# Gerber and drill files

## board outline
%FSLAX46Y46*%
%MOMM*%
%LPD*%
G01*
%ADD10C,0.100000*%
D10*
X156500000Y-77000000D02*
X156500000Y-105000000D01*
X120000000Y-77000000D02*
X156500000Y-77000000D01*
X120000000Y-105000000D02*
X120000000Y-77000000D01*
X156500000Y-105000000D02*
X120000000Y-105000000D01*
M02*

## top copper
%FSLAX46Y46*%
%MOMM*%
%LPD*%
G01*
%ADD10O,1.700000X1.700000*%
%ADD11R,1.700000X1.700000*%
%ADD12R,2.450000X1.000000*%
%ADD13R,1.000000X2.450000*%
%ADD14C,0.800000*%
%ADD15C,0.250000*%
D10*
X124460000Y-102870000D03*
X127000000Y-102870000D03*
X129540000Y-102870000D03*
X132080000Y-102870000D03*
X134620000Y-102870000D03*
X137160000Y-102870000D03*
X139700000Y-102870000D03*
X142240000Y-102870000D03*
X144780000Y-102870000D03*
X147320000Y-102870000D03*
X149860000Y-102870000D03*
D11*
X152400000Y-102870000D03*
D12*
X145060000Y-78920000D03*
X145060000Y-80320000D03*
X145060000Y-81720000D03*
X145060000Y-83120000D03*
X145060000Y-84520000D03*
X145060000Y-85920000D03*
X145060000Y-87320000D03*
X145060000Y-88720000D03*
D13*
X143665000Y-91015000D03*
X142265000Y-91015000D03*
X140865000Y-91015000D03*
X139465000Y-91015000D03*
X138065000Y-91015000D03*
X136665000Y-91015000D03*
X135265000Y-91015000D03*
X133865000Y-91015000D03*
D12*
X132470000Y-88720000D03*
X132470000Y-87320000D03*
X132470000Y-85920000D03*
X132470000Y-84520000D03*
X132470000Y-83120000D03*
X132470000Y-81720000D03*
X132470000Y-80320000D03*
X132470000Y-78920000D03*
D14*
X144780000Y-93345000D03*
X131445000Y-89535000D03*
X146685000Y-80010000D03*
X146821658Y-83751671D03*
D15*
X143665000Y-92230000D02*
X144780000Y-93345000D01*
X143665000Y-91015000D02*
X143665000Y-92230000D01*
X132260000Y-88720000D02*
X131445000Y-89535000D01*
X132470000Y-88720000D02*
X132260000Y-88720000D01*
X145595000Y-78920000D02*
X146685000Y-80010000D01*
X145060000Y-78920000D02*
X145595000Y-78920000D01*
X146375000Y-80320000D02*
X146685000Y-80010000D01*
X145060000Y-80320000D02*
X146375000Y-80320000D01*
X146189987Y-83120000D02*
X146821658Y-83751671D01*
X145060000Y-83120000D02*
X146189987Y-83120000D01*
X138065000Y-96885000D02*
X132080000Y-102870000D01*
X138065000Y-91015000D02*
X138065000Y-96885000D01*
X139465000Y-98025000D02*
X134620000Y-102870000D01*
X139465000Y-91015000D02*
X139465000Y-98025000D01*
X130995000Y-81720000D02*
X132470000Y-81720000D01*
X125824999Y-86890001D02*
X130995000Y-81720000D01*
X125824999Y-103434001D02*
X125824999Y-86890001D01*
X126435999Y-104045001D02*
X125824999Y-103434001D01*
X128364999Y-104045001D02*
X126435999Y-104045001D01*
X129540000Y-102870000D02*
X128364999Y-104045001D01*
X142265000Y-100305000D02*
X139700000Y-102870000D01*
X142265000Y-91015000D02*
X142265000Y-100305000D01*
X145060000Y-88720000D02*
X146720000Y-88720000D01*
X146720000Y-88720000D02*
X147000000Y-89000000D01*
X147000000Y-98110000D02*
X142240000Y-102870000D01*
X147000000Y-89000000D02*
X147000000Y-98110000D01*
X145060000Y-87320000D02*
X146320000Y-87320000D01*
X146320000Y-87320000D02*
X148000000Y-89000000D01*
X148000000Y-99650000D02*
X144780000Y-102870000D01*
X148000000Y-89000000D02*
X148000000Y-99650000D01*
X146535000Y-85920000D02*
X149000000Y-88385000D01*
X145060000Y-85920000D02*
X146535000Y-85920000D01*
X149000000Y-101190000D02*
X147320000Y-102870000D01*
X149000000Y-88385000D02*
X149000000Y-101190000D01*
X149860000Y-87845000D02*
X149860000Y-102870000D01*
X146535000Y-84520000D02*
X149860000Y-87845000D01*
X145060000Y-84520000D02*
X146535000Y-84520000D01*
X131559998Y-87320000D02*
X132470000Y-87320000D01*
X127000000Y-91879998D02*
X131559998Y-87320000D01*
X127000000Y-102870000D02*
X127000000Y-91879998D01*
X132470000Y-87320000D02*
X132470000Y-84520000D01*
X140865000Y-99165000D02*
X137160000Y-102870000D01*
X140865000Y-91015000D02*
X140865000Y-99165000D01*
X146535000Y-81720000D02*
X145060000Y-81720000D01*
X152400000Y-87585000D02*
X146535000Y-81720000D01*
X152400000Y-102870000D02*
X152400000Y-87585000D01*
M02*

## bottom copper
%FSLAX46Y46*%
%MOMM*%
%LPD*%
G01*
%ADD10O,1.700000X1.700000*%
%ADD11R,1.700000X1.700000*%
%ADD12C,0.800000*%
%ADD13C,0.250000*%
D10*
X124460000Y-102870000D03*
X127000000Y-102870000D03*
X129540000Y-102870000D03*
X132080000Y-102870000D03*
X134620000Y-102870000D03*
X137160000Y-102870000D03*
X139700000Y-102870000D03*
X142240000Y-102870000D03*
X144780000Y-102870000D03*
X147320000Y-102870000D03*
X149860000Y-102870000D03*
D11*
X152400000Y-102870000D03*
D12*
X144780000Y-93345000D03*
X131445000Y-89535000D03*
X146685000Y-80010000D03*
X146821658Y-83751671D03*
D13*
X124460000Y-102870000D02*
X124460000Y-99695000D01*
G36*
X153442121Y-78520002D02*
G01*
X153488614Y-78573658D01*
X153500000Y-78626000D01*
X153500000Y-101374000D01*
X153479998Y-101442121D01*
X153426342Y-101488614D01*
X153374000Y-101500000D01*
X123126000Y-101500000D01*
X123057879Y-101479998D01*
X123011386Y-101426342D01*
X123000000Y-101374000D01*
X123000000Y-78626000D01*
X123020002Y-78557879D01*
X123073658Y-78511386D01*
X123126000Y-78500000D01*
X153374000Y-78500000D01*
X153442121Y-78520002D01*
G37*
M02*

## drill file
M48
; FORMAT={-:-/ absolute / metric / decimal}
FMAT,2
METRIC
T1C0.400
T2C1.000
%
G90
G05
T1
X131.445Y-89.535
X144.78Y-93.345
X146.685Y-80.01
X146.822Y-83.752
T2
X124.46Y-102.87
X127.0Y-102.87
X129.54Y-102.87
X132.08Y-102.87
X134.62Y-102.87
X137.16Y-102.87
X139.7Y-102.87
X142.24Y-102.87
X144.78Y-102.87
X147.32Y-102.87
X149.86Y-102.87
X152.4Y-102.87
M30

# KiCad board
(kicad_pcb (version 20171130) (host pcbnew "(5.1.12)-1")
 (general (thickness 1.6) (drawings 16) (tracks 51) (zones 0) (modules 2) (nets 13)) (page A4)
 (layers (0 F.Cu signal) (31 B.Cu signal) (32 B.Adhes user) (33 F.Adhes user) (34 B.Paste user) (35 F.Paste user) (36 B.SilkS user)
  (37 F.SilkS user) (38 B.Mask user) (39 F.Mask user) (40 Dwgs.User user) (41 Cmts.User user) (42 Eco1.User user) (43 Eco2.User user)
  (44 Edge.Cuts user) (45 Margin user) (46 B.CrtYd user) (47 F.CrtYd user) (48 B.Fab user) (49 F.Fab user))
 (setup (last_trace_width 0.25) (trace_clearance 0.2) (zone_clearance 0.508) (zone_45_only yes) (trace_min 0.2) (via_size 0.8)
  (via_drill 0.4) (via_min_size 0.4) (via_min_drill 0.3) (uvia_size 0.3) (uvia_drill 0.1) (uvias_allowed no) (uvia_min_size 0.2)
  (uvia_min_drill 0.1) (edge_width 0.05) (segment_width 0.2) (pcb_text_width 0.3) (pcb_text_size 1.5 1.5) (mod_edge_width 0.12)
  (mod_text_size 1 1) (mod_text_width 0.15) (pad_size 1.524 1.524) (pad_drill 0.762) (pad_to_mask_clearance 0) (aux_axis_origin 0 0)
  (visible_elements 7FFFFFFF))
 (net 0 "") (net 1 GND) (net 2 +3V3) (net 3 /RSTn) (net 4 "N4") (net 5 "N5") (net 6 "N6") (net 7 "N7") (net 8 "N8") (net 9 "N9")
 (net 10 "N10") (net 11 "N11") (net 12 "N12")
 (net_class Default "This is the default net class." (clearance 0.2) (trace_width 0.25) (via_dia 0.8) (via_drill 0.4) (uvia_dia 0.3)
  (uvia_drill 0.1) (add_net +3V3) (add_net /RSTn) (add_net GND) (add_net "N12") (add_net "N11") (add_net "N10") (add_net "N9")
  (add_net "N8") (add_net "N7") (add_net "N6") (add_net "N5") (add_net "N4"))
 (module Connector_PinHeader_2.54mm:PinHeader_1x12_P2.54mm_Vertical (layer F.Cu) (at 152.4 102.87 270)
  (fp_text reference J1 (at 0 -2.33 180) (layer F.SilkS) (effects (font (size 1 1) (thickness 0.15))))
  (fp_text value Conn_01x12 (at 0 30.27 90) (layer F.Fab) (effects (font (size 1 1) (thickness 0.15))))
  (pad 12 thru_hole oval (at 0 27.94 270) (size 1.7 1.7) (drill 1) (layers *.Cu *.Mask) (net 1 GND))
  (pad 11 thru_hole oval (at 0 25.4 270) (size 1.7 1.7) (drill 1) (layers *.Cu *.Mask) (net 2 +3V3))
  (pad 10 thru_hole oval (at 0 22.86 270) (size 1.7 1.7) (drill 1) (layers *.Cu *.Mask) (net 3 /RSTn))
  (pad 9 thru_hole oval (at 0 20.32 270) (size 1.7 1.7) (drill 1) (layers *.Cu *.Mask) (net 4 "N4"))
  (pad 8 thru_hole oval (at 0 17.78 270) (size 1.7 1.7) (drill 1) (layers *.Cu *.Mask) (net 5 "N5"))
  (pad 7 thru_hole oval (at 0 15.24 270) (size 1.7 1.7) (drill 1) (layers *.Cu *.Mask) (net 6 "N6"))
  (pad 6 thru_hole oval (at 0 12.7 270) (size 1.7 1.7) (drill 1) (layers *.Cu *.Mask) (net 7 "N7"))
  (pad 5 thru_hole oval (at 0 10.16 270) (size 1.7 1.7) (drill 1) (layers *.Cu *.Mask) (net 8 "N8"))
  (pad 4 thru_hole oval (at 0 7.62 270) (size 1.7 1.7) (drill 1) (layers *.Cu *.Mask) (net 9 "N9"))
  (pad 3 thru_hole oval (at 0 5.08 270) (size 1.7 1.7) (drill 1) (layers *.Cu *.Mask) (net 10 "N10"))
  (pad 2 thru_hole oval (at 0 2.54 270) (size 1.7 1.7) (drill 1) (layers *.Cu *.Mask) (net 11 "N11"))
  (pad 1 thru_hole rect (at 0 0 270) (size 1.7 1.7) (drill 1) (layers *.Cu *.Mask) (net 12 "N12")))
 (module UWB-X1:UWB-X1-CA (layer F.Cu) (at 138.765 83.82)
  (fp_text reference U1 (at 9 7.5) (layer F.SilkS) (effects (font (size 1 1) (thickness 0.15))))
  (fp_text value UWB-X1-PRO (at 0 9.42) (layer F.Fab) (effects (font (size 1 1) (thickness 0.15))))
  (pad 24 smd rect (at 6.295 -4.9 90) (size 1 2.45) (layers F.Cu F.Paste F.Mask) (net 1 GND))
  (pad 23 smd rect (at 6.295 -3.5 90) (size 1 2.45) (layers F.Cu F.Paste F.Mask) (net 1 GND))
  (pad 22 smd rect (at 6.295 -2.1 90) (size 1 2.45) (layers F.Cu F.Paste F.Mask) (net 12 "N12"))
  (pad 21 smd rect (at 6.295 -0.7 90) (size 1 2.45) (layers F.Cu F.Paste F.Mask) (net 1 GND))
  (pad 20 smd rect (at 6.295 0.7 90) (size 1 2.45) (layers F.Cu F.Paste F.Mask) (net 11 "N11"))
  (pad 19 smd rect (at 6.295 2.1 90) (size 1 2.45) (layers F.Cu F.Paste F.Mask) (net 10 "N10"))
  (pad 18 smd rect (at 6.295 3.5 90) (size 1 2.45) (layers F.Cu F.Paste F.Mask) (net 9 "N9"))
  (pad 17 smd rect (at 6.295 4.9 90) (size 1 2.45) (layers F.Cu F.Paste F.Mask) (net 8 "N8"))
  (pad 16 smd rect (at 4.9 7.195) (size 1 2.45) (layers F.Cu F.Paste F.Mask) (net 1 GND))
  (pad 15 smd rect (at 3.5 7.195) (size 1 2.45) (layers F.Cu F.Paste F.Mask) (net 7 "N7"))
  (pad 14 smd rect (at 2.1 7.195) (size 1 2.45) (layers F.Cu F.Paste F.Mask) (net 6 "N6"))
  (pad 13 smd rect (at 0.7 7.195) (size 1 2.45) (layers F.Cu F.Paste F.Mask) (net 5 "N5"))
  (pad 12 smd rect (at -0.7 7.195) (size 1 2.45) (layers F.Cu F.Paste F.Mask) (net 4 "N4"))
  (pad 11 smd rect (at -2.1 7.195) (size 1 2.45) (layers F.Cu F.Paste F.Mask))
  (pad 10 smd rect (at -3.5 7.195) (size 1 2.45) (layers F.Cu F.Paste F.Mask))
  (pad 9 smd rect (at -4.9 7.195) (size 1 2.45) (layers F.Cu F.Paste F.Mask))
  (pad 8 smd rect (at -6.295 4.9 90) (size 1 2.45) (layers F.Cu F.Paste F.Mask) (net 1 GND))
  (pad 7 smd rect (at -6.295 3.5 90) (size 1 2.45) (layers F.Cu F.Paste F.Mask) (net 2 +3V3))
  (pad 6 smd rect (at -6.295 2.1 90) (size 1 2.45) (layers F.Cu F.Paste F.Mask) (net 2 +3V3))
  (pad 5 smd rect (at -6.295 0.7 90) (size 1 2.45) (layers F.Cu F.Paste F.Mask) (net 2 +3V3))
  (pad 4 smd rect (at -6.295 -0.7 90) (size 1 2.45) (layers F.Cu F.Paste F.Mask))
  (pad 3 smd rect (at -6.295 -2.1 90) (size 1 2.45) (layers F.Cu F.Paste F.Mask) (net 3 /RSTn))
  (pad 2 smd rect (at -6.295 -3.5 90) (size 1 2.45) (layers F.Cu F.Paste F.Mask))
  (pad 1 smd rect (at -6.295 -4.9 90) (size 1 2.45) (layers F.Cu F.Paste F.Mask)))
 (gr_line (start 156.5 77) (end 156.5 105) (layer Edge.Cuts) (width 0.1))
 (gr_line (start 120 77) (end 156.5 77) (layer Edge.Cuts) (width 0.1))
 (gr_line (start 120 105) (end 120 77) (layer Edge.Cuts) (width 0.1))
 (gr_line (start 156.5 105) (end 120 105) (layer Edge.Cuts) (width 0.1))
 (via (at 144.78 93.345) (size 0.8) (drill 0.4) (layers F.Cu B.Cu) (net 1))
 (segment (start 143.665 92.23) (end 144.78 93.345) (width 0.25) (layer F.Cu) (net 1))
 (segment (start 143.665 91.015) (end 143.665 92.23) (width 0.25) (layer F.Cu) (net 1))
 (segment (start 132.26 88.72) (end 131.445 89.535) (width 0.25) (layer F.Cu) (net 1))
 (via (at 131.445 89.535) (size 0.8) (drill 0.4) (layers F.Cu B.Cu) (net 1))
 (segment (start 132.47 88.72) (end 132.26 88.72) (width 0.25) (layer F.Cu) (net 1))
 (via (at 146.685 80.01) (size 0.8) (drill 0.4) (layers F.Cu B.Cu) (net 1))
 (segment (start 145.595 78.92) (end 146.685 80.01) (width 0.25) (layer F.Cu) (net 1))
 (segment (start 145.06 78.92) (end 145.595 78.92) (width 0.25) (layer F.Cu) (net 1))
 (segment (start 146.375 80.32) (end 146.685 80.01) (width 0.25) (layer F.Cu) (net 1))
 (segment (start 145.06 80.32) (end 146.375 80.32) (width 0.25) (layer F.Cu) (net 1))
 (via (at 146.821658 83.751671) (size 0.8) (drill 0.4) (layers F.Cu B.Cu) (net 1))
 (segment (start 146.189987 83.12) (end 146.821658 83.751671) (width 0.25) (layer F.Cu) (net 1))
 (segment (start 145.06 83.12) (end 146.189987 83.12) (width 0.25) (layer F.Cu) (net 1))
 (segment (start 124.46 102.87) (end 124.46 99.695) (width 0.25) (layer B.Cu) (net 1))
 (segment (start 138.065 96.885) (end 132.08 102.87) (width 0.25) (layer F.Cu) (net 4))
 (segment (start 138.065 91.015) (end 138.065 96.885) (width 0.25) (layer F.Cu) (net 4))
 (segment (start 139.465 98.025) (end 134.62 102.87) (width 0.25) (layer F.Cu) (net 5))
 (segment (start 139.465 91.015) (end 139.465 98.025) (width 0.25) (layer F.Cu) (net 5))
 (segment (start 130.995 81.72) (end 132.47 81.72) (width 0.25) (layer F.Cu) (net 3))
 (segment (start 125.824999 86.890001) (end 130.995 81.72) (width 0.25) (layer F.Cu) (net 3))
 (segment (start 125.824999 103.434001) (end 125.824999 86.890001) (width 0.25) (layer F.Cu) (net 3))
 (segment (start 126.435999 104.045001) (end 125.824999 103.434001) (width 0.25) (layer F.Cu) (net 3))
 (segment (start 128.364999 104.045001) (end 126.435999 104.045001) (width 0.25) (layer F.Cu) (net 3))
 (segment (start 129.54 102.87) (end 128.364999 104.045001) (width 0.25) (layer F.Cu) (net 3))
 (segment (start 142.265 100.305) (end 139.7 102.87) (width 0.25) (layer F.Cu) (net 7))
 (segment (start 142.265 91.015) (end 142.265 100.305) (width 0.25) (layer F.Cu) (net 7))
 (segment (start 145.06 88.72) (end 146.72 88.72) (width 0.25) (layer F.Cu) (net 8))
 (segment (start 146.72 88.72) (end 147 89) (width 0.25) (layer F.Cu) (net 8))
 (segment (start 147 98.11) (end 142.24 102.87) (width 0.25) (layer F.Cu) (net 8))
 (segment (start 147 89) (end 147 98.11) (width 0.25) (layer F.Cu) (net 8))
 (segment (start 145.06 87.32) (end 146.32 87.32) (width 0.25) (layer F.Cu) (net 9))
 (segment (start 146.32 87.32) (end 148 89) (width 0.25) (layer F.Cu) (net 9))
 (segment (start 148 99.65) (end 144.78 102.87) (width 0.25) (layer F.Cu) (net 9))
 (segment (start 148 89) (end 148 99.65) (width 0.25) (layer F.Cu) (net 9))
 (segment (start 146.535 85.92) (end 149 88.385) (width 0.25) (layer F.Cu) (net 10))
 (segment (start 145.06 85.92) (end 146.535 85.92) (width 0.25) (layer F.Cu) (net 10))
 (segment (start 149 101.19) (end 147.32 102.87) (width 0.25) (layer F.Cu) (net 10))
 (segment (start 149 88.385) (end 149 101.19) (width 0.25) (layer F.Cu) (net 10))
 (segment (start 149.86 87.845) (end 149.86 102.87) (width 0.25) (layer F.Cu) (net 11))
 (segment (start 146.535 84.52) (end 149.86 87.845) (width 0.25) (layer F.Cu) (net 11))
 (segment (start 145.06 84.52) (end 146.535 84.52) (width 0.25) (layer F.Cu) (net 11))
 (segment (start 131.559998 87.32) (end 132.47 87.32) (width 0.25) (layer F.Cu) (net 2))
 (segment (start 127 91.879998) (end 131.559998 87.32) (width 0.25) (layer F.Cu) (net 2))
 (segment (start 127 102.87) (end 127 91.879998) (width 0.25) (layer F.Cu) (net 2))
 (segment (start 132.47 87.32) (end 132.47 84.52) (width 0.25) (layer F.Cu) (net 2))
 (segment (start 140.865 99.165) (end 137.16 102.87) (width 0.25) (layer F.Cu) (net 6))
 (segment (start 140.865 91.015) (end 140.865 99.165) (width 0.25) (layer F.Cu) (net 6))
 (segment (start 146.535 81.72) (end 145.06 81.72) (width 0.25) (layer F.Cu) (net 12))
 (segment (start 152.4 87.585) (end 146.535 81.72) (width 0.25) (layer F.Cu) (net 12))
 (segment (start 152.4 102.87) (end 152.4 87.585) (width 0.25) (layer F.Cu) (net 12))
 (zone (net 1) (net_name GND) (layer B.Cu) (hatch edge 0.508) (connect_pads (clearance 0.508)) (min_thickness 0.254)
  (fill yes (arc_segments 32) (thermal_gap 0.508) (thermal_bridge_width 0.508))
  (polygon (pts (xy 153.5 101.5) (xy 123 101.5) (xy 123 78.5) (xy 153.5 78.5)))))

